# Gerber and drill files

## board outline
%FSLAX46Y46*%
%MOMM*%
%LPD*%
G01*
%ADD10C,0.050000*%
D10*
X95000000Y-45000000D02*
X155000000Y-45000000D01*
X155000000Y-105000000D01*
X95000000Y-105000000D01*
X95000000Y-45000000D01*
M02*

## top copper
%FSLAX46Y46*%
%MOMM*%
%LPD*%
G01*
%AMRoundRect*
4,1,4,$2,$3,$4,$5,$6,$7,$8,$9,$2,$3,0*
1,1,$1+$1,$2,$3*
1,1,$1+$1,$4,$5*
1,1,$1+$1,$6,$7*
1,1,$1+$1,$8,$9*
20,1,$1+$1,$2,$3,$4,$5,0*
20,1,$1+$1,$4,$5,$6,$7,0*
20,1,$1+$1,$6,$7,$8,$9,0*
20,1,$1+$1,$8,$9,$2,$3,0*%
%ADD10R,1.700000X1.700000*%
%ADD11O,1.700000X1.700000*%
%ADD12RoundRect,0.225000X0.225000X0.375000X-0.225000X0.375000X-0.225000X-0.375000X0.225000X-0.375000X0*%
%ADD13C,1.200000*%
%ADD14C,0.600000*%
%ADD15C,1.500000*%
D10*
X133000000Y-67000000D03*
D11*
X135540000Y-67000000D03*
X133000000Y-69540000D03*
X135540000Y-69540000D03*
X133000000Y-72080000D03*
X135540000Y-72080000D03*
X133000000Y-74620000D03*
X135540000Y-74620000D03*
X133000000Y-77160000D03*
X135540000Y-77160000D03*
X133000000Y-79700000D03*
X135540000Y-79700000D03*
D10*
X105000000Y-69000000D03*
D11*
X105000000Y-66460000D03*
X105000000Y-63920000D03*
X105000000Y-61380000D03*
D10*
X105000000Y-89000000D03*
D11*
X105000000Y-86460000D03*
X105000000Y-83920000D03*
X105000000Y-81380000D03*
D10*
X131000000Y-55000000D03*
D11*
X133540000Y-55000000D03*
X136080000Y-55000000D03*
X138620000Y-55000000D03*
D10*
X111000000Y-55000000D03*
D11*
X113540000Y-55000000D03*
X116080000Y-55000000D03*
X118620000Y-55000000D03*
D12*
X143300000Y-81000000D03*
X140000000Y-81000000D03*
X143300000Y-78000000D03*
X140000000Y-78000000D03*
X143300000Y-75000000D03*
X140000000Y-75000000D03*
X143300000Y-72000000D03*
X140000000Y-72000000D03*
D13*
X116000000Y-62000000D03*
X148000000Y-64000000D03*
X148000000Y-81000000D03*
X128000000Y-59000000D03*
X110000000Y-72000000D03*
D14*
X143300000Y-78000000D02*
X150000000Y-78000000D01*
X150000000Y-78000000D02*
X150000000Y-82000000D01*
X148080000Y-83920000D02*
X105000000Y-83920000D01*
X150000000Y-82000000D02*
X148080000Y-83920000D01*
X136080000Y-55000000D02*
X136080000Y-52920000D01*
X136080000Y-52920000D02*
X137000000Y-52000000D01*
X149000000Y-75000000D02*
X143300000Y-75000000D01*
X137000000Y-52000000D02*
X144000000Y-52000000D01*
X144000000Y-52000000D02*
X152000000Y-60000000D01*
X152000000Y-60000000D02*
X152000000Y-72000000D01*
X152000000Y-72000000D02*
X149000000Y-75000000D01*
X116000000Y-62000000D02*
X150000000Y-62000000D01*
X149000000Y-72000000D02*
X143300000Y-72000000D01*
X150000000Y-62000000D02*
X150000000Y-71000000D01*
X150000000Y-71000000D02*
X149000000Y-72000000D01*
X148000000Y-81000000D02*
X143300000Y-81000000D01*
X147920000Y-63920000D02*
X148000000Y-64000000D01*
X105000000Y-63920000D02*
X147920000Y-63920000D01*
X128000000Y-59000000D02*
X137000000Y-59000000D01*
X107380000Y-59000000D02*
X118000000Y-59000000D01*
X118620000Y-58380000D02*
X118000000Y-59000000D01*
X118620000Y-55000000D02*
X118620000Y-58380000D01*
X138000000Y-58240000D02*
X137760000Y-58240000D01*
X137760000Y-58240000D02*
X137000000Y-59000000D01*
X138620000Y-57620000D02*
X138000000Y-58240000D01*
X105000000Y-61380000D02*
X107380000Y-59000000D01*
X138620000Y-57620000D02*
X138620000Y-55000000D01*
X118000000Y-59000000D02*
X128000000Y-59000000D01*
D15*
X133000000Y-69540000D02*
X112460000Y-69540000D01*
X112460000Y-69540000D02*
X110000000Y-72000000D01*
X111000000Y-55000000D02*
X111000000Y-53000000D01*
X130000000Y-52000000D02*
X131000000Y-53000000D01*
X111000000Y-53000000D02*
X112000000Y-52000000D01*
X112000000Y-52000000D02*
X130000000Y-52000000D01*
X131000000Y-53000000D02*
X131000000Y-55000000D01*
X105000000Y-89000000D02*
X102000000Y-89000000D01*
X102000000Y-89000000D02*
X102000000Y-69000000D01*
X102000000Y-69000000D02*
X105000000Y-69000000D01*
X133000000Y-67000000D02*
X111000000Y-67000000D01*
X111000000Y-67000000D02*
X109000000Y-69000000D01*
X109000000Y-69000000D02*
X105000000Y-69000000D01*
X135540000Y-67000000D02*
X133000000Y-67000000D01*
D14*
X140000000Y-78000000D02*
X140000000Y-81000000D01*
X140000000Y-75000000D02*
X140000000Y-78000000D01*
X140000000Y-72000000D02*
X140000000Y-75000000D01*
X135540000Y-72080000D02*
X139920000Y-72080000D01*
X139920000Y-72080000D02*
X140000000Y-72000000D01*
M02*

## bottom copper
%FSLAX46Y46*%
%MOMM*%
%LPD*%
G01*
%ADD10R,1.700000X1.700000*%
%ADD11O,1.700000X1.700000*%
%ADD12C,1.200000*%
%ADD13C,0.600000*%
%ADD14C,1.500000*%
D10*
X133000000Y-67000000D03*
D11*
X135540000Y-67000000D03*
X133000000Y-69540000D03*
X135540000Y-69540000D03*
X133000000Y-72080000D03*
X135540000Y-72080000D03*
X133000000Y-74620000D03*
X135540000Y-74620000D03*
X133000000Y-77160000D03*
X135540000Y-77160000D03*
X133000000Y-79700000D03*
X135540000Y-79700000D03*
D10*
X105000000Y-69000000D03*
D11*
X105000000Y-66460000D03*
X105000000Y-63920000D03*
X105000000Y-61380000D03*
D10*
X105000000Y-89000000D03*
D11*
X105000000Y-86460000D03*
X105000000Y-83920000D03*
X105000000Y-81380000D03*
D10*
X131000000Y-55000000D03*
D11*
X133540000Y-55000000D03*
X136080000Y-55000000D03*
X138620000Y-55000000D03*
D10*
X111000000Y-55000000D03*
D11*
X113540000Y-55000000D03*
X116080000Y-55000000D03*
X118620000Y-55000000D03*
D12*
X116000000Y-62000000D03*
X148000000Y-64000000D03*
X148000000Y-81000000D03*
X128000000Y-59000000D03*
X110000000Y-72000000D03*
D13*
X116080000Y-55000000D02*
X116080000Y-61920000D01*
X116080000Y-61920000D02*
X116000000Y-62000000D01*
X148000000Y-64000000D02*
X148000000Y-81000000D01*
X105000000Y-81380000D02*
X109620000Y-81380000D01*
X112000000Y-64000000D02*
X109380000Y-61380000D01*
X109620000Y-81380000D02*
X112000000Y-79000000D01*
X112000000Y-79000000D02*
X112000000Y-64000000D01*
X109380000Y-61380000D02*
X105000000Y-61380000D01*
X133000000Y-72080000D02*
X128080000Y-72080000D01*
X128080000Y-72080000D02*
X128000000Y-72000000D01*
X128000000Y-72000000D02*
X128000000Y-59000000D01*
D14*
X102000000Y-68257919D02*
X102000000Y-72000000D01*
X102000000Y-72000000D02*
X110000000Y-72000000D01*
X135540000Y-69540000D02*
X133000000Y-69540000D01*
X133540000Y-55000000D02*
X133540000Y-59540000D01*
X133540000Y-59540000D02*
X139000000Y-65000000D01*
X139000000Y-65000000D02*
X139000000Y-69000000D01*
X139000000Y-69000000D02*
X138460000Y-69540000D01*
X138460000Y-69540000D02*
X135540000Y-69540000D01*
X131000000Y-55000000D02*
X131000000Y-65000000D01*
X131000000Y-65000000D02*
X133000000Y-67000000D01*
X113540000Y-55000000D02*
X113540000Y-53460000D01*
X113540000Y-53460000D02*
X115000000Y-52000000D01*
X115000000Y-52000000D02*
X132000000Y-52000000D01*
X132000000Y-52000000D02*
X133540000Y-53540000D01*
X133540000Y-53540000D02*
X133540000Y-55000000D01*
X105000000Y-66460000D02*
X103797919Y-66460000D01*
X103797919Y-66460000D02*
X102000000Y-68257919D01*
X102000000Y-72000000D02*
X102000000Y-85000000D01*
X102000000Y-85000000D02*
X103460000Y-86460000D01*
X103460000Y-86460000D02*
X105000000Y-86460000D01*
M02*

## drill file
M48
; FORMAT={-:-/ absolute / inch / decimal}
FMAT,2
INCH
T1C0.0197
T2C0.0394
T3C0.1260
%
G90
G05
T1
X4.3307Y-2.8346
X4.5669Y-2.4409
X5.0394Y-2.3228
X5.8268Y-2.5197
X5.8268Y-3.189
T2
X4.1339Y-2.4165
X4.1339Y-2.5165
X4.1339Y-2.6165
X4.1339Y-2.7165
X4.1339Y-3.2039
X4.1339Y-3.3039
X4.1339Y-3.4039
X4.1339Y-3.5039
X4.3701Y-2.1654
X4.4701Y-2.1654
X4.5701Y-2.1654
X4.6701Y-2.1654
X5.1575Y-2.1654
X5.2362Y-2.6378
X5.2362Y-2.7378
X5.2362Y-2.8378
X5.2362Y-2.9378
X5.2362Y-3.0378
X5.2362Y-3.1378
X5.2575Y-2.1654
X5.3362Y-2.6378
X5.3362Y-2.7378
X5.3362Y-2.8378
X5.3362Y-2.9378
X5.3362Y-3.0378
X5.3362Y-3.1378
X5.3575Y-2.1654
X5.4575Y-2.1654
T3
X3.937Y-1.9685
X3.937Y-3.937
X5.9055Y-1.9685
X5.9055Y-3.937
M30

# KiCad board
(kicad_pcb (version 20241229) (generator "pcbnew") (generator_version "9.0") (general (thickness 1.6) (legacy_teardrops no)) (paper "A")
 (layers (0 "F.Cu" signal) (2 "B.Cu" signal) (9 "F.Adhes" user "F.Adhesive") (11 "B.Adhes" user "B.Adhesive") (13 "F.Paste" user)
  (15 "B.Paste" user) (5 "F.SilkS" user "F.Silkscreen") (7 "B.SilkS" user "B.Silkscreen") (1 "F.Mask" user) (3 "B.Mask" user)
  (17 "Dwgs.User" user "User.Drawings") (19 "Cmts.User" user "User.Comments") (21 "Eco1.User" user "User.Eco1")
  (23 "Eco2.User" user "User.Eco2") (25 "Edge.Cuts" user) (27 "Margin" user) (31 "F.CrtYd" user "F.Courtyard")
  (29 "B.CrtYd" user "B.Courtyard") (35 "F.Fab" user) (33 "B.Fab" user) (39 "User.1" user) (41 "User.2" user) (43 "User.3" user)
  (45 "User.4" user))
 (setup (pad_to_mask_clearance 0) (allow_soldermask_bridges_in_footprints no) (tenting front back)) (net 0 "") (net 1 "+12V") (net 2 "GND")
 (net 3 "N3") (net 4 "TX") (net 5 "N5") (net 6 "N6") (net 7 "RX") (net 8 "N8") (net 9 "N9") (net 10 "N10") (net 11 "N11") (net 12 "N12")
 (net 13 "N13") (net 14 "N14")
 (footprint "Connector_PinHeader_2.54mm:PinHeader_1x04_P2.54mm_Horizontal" (layer "F.Cu") (at 131 55 90)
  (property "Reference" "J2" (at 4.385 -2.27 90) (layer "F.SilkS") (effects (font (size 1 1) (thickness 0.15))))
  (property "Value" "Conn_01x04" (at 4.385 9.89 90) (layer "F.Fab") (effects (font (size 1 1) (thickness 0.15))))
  (pad "1" thru_hole rect (at 0 0 90) (size 1.7 1.7) (drill 1) (layers "*.Cu" "*.Mask") (remove_unused_layers no) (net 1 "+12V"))
  (pad "2" thru_hole oval (at 0 2.54 90) (size 1.7 1.7) (drill 1) (layers "*.Cu" "*.Mask") (remove_unused_layers no) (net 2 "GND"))
  (pad "3" thru_hole oval (at 0 5.08 90) (size 1.7 1.7) (drill 1) (layers "*.Cu" "*.Mask") (remove_unused_layers no) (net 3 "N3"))
  (pad "4" thru_hole oval (at 0 7.62 90) (size 1.7 1.7) (drill 1) (layers "*.Cu" "*.Mask") (remove_unused_layers no) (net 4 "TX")))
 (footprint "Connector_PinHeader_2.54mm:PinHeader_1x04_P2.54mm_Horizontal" (layer "F.Cu") (at 105 89 180)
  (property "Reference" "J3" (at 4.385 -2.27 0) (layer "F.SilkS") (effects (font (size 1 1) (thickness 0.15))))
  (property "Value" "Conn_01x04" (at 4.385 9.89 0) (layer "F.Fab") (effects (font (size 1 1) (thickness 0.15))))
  (pad "1" thru_hole rect (at 0 0 180) (size 1.7 1.7) (drill 1) (layers "*.Cu" "*.Mask") (remove_unused_layers no) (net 1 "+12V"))
  (pad "2" thru_hole oval (at 0 2.54 180) (size 1.7 1.7) (drill 1) (layers "*.Cu" "*.Mask") (remove_unused_layers no) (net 2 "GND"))
  (pad "3" thru_hole oval (at 0 5.08 180) (size 1.7 1.7) (drill 1) (layers "*.Cu" "*.Mask") (remove_unused_layers no) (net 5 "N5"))
  (pad "4" thru_hole oval (at 0 7.62 180) (size 1.7 1.7) (drill 1) (layers "*.Cu" "*.Mask") (remove_unused_layers no) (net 4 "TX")))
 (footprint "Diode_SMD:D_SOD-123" (layer "F.Cu") (at 141.65 81 180)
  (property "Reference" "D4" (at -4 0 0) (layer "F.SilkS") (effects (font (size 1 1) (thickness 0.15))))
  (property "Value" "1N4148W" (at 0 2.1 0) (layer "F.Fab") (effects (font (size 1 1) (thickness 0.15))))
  (pad "1" smd roundrect (at -1.65 0 180) (size 0.9 1.2) (layers "F.Cu" "F.Mask" "F.Paste") (roundrect_rratio 0.25) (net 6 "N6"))
  (pad "2" smd roundrect (at 1.65 0 180) (size 0.9 1.2) (layers "F.Cu" "F.Mask" "F.Paste") (roundrect_rratio 0.25) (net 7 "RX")))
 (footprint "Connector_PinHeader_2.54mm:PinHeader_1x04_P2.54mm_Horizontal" (layer "F.Cu") (at 105 69 180)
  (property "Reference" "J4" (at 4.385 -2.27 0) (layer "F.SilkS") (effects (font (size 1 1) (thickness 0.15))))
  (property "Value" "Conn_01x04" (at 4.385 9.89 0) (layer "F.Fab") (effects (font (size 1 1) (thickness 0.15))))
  (pad "1" thru_hole rect (at 0 0 180) (size 1.7 1.7) (drill 1) (layers "*.Cu" "*.Mask") (remove_unused_layers no) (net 1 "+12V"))
  (pad "2" thru_hole oval (at 0 2.54 180) (size 1.7 1.7) (drill 1) (layers "*.Cu" "*.Mask") (remove_unused_layers no) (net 2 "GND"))
  (pad "3" thru_hole oval (at 0 5.08 180) (size 1.7 1.7) (drill 1) (layers "*.Cu" "*.Mask") (remove_unused_layers no) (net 6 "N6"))
  (pad "4" thru_hole oval (at 0 7.62 180) (size 1.7 1.7) (drill 1) (layers "*.Cu" "*.Mask") (remove_unused_layers no) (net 4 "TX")))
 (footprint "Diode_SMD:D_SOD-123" (layer "F.Cu") (at 141.65 75 180)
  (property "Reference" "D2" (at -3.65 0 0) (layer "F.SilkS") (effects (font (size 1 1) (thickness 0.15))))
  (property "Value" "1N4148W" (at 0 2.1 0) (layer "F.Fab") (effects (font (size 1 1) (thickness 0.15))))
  (pad "1" smd roundrect (at -1.65 0 180) (size 0.9 1.2) (layers "F.Cu" "F.Mask" "F.Paste") (roundrect_rratio 0.25) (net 3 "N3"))
  (pad "2" smd roundrect (at 1.65 0 180) (size 0.9 1.2) (layers "F.Cu" "F.Mask" "F.Paste") (roundrect_rratio 0.25) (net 7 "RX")))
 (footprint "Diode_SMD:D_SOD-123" (layer "F.Cu") (at 141.65 72 180)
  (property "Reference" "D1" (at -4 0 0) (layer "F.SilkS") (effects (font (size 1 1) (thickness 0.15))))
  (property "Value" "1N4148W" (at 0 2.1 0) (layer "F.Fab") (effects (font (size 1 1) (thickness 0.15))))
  (pad "1" smd roundrect (at -1.65 0 180) (size 0.9 1.2) (layers "F.Cu" "F.Mask" "F.Paste") (roundrect_rratio 0.25) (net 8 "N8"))
  (pad "2" smd roundrect (at 1.65 0 180) (size 0.9 1.2) (layers "F.Cu" "F.Mask" "F.Paste") (roundrect_rratio 0.25) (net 7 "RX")))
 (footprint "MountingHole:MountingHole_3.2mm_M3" (layer "F.Cu") (at 150 100)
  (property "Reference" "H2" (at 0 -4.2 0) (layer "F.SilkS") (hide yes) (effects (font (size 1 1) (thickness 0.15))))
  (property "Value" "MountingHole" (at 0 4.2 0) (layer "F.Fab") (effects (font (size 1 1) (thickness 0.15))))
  (pad "" np_thru_hole circle (at 0 0) (size 3.2 3.2) (drill 3.2) (layers "*.Cu" "*.Mask")))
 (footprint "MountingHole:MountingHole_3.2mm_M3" (layer "F.Cu") (at 100 50)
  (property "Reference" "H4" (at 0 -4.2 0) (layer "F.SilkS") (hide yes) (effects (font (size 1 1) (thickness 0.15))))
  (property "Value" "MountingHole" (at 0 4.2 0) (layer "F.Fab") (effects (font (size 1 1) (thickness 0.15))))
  (pad "" np_thru_hole circle (at 0 0) (size 3.2 3.2) (drill 3.2) (layers "*.Cu" "*.Mask")))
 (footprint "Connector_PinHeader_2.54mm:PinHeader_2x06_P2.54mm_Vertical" (layer "F.Cu") (at 133 67)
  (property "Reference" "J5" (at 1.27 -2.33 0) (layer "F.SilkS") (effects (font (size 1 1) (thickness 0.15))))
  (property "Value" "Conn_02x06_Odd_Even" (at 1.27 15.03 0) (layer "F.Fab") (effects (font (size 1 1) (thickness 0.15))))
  (pad "1" thru_hole rect (at 0 0) (size 1.7 1.7) (drill 1) (layers "*.Cu" "*.Mask") (remove_unused_layers no) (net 1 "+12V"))
  (pad "2" thru_hole oval (at 2.54 0) (size 1.7 1.7) (drill 1) (layers "*.Cu" "*.Mask") (remove_unused_layers no) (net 1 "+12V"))
  (pad "3" thru_hole oval (at 0 2.54) (size 1.7 1.7) (drill 1) (layers "*.Cu" "*.Mask") (remove_unused_layers no) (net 2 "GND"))
  (pad "4" thru_hole oval (at 2.54 2.54) (size 1.7 1.7) (drill 1) (layers "*.Cu" "*.Mask") (remove_unused_layers no) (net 2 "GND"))
  (pad "5" thru_hole oval (at 0 5.08) (size 1.7 1.7) (drill 1) (layers "*.Cu" "*.Mask") (remove_unused_layers no) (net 4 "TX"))
  (pad "6" thru_hole oval (at 2.54 5.08) (size 1.7 1.7) (drill 1) (layers "*.Cu" "*.Mask") (remove_unused_layers no) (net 7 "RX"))
  (pad "7" thru_hole oval (at 0 7.62) (size 1.7 1.7) (drill 1) (layers "*.Cu" "*.Mask") (remove_unused_layers no) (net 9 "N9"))
  (pad "8" thru_hole oval (at 2.54 7.62) (size 1.7 1.7) (drill 1) (layers "*.Cu" "*.Mask") (remove_unused_layers no) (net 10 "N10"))
  (pad "9" thru_hole oval (at 0 10.16) (size 1.7 1.7) (drill 1) (layers "*.Cu" "*.Mask") (remove_unused_layers no) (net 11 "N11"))
  (pad "10" thru_hole oval (at 2.54 10.16) (size 1.7 1.7) (drill 1) (layers "*.Cu" "*.Mask") (remove_unused_layers no) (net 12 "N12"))
  (pad "11" thru_hole oval (at 0 12.7) (size 1.7 1.7) (drill 1) (layers "*.Cu" "*.Mask") (remove_unused_layers no) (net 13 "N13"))
  (pad "12" thru_hole oval (at 2.54 12.7) (size 1.7 1.7) (drill 1) (layers "*.Cu" "*.Mask") (remove_unused_layers no) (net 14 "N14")))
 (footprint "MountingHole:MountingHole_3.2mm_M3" (layer "F.Cu") (at 100 100)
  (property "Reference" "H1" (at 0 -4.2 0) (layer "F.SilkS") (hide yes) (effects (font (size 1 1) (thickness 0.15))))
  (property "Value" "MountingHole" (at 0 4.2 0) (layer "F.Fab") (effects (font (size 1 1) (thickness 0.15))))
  (pad "" np_thru_hole circle (at 0 0) (size 3.2 3.2) (drill 3.2) (layers "*.Cu" "*.Mask")))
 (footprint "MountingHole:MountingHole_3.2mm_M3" (layer "F.Cu") (at 150 50)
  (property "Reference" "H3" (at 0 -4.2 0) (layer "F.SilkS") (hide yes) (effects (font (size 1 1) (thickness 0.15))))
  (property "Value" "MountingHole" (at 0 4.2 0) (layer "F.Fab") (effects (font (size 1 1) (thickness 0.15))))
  (pad "" np_thru_hole circle (at 0 0) (size 3.2 3.2) (drill 3.2) (layers "*.Cu" "*.Mask")))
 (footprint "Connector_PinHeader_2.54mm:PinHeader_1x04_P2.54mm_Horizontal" (layer "F.Cu") (at 111 55 90)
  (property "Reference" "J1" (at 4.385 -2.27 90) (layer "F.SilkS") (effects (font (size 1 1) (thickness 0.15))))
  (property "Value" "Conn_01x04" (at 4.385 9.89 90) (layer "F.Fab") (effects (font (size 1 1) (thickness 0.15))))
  (pad "1" thru_hole rect (at 0 0 90) (size 1.7 1.7) (drill 1) (layers "*.Cu" "*.Mask") (remove_unused_layers no) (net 1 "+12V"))
  (pad "2" thru_hole oval (at 0 2.54 90) (size 1.7 1.7) (drill 1) (layers "*.Cu" "*.Mask") (remove_unused_layers no) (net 2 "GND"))
  (pad "3" thru_hole oval (at 0 5.08 90) (size 1.7 1.7) (drill 1) (layers "*.Cu" "*.Mask") (remove_unused_layers no) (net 8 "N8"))
  (pad "4" thru_hole oval (at 0 7.62 90) (size 1.7 1.7) (drill 1) (layers "*.Cu" "*.Mask") (remove_unused_layers no) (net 4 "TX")))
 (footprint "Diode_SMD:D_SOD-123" (layer "F.Cu") (at 141.65 78 180)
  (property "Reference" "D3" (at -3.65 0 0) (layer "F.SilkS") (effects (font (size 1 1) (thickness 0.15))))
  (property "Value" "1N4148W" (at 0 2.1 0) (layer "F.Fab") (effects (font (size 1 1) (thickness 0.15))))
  (pad "1" smd roundrect (at -1.65 0 180) (size 0.9 1.2) (layers "F.Cu" "F.Mask" "F.Paste") (roundrect_rratio 0.25) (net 5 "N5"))
  (pad "2" smd roundrect (at 1.65 0 180) (size 0.9 1.2) (layers "F.Cu" "F.Mask" "F.Paste") (roundrect_rratio 0.25) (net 7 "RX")))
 (gr_rect (start 95 45) (end 155 105) (stroke (width 0.05) (type default)) (fill no) (layer "Edge.Cuts"))
 (segment (start 116 62) (end 150 62) (width 0.6) (layer "F.Cu") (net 8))
 (segment (start 150 62) (end 150 71) (width 0.6) (layer "F.Cu") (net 8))
 (segment (start 149 72) (end 143.3 72) (width 0.6) (layer "F.Cu") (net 8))
 (segment (start 150 71) (end 149 72) (width 0.6) (layer "F.Cu") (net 8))
 (via (at 116 62) (size 1.2) (drill 0.5) (layers "F.Cu" "B.Cu") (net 8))
 (segment (start 116.08 55) (end 116.08 61.92) (width 0.6) (layer "B.Cu") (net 8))
 (segment (start 116.08 61.92) (end 116 62) (width 0.6) (layer "B.Cu") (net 8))
 (segment (start 140 75) (end 140 78) (width 0.6) (layer "F.Cu") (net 7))
 (segment (start 140 78) (end 140 81) (width 0.6) (layer "F.Cu") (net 7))
 (segment (start 135.54 72.08) (end 139.92 72.08) (width 0.6) (layer "F.Cu") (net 7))
 (segment (start 139.92 72.08) (end 140 72) (width 0.6) (layer "F.Cu") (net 7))
 (segment (start 140 72) (end 140 75) (width 0.6) (layer "F.Cu") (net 7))
 (segment (start 136.08 55) (end 136.08 52.92) (width 0.6) (layer "F.Cu") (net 3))
 (segment (start 152 72) (end 149 75) (width 0.6) (layer "F.Cu") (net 3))
 (segment (start 136.08 52.92) (end 137 52) (width 0.6) (layer "F.Cu") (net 3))
 (segment (start 144 52) (end 152 60) (width 0.6) (layer "F.Cu") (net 3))
 (segment (start 152 60) (end 152 72) (width 0.6) (layer "F.Cu") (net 3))
 (segment (start 137 52) (end 144 52) (width 0.6) (layer "F.Cu") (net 3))
 (segment (start 149 75) (end 143.3 75) (width 0.6) (layer "F.Cu") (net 3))
 (segment (start 150 82) (end 148.08 83.92) (width 0.6) (layer "F.Cu") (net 5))
 (segment (start 150 78) (end 150 82) (width 0.6) (layer "F.Cu") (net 5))
 (segment (start 148.08 83.92) (end 105 83.92) (width 0.6) (layer "F.Cu") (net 5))
 (segment (start 143.3 78) (end 150 78) (width 0.6) (layer "F.Cu") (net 5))
 (segment (start 147.92 63.92) (end 148 64) (width 0.6) (layer "F.Cu") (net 6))
 (segment (start 105 63.92) (end 147.92 63.92) (width 0.6) (layer "F.Cu") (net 6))
 (segment (start 148 81) (end 143.3 81) (width 0.6) (layer "F.Cu") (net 6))
 (via (at 148 64) (size 1.2) (drill 0.5) (layers "F.Cu" "B.Cu") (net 6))
 (via (at 148 81) (size 1.2) (drill 0.5) (layers "F.Cu" "B.Cu") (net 6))
 (segment (start 148 64) (end 148 81) (width 0.6) (layer "B.Cu") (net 6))
 (segment (start 105 89) (end 102 89) (width 1.5) (layer "F.Cu") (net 1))
 (segment (start 135.54 67) (end 133 67) (width 1.5) (layer "F.Cu") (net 1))
 (segment (start 102 69) (end 105 69) (width 1.5) (layer "F.Cu") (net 1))
 (segment (start 102 89) (end 102 69) (width 1.5) (layer "F.Cu") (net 1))
 (segment (start 131 53) (end 131 55) (width 1.5) (layer "F.Cu") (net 1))
 (segment (start 112 52) (end 130 52) (width 1.5) (layer "F.Cu") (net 1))
 (segment (start 133 67) (end 111 67) (width 1.5) (layer "F.Cu") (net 1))
 (segment (start 111 67) (end 109 69) (width 1.5) (layer "F.Cu") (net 1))
 (segment (start 111 55) (end 111 53) (width 1.5) (layer "F.Cu") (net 1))
 (segment (start 109 69) (end 105 69) (width 1.5) (layer "F.Cu") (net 1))
 (segment (start 130 52) (end 131 53) (width 1.5) (layer "F.Cu") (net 1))
 (segment (start 111 53) (end 112 52) (width 1.5) (layer "F.Cu") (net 1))
 (segment (start 131 55) (end 131 65) (width 1.5) (layer "B.Cu") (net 1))
 (segment (start 131 65) (end 133 67) (width 1.5) (layer "B.Cu") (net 1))
 (segment (start 138.62 57.62) (end 138.62 55) (width 0.6) (layer "F.Cu") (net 4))
 (segment (start 105 61.38) (end 107.38 59) (width 0.6) (layer "F.Cu") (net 4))
 (segment (start 138.62 57.62) (end 138 58.24) (width 0.6) (layer "F.Cu") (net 4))
 (segment (start 137.76 58.24) (end 137 59) (width 0.6) (layer "F.Cu") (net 4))
 (segment (start 138 58.24) (end 137.76 58.24) (width 0.6) (layer "F.Cu") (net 4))
 (segment (start 118.62 55) (end 118.62 58.38) (width 0.6) (layer "F.Cu") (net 4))
 (segment (start 118 59) (end 128 59) (width 0.6) (layer "F.Cu") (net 4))
 (segment (start 128 59) (end 137 59) (width 0.6) (layer "F.Cu") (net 4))
 (segment (start 107.38 59) (end 118 59) (width 0.6) (layer "F.Cu") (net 4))
 (segment (start 118.62 58.38) (end 118 59) (width 0.6) (layer "F.Cu") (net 4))
 (via (at 128 59) (size 1.2) (drill 0.5) (layers "F.Cu" "B.Cu") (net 4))
 (segment (start 112 79) (end 112 64) (width 0.6) (layer "B.Cu") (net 4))
 (segment (start 105 81.38) (end 109.62 81.38) (width 0.6) (layer "B.Cu") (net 4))
 (segment (start 128 72) (end 128 59) (width 0.6) (layer "B.Cu") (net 4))
 (segment (start 109.62 81.38) (end 112 79) (width 0.6) (layer "B.Cu") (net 4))
 (segment (start 112 64) (end 109.38 61.38) (width 0.6) (layer "B.Cu") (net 4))
 (segment (start 133 72.08) (end 128.08 72.08) (width 0.6) (layer "B.Cu") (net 4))
 (segment (start 109.38 61.38) (end 105 61.38) (width 0.6) (layer "B.Cu") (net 4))
 (segment (start 128.08 72.08) (end 128 72) (width 0.6) (layer "B.Cu") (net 4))
 (segment (start 133 69.54) (end 112.46 69.54) (width 1.5) (layer "F.Cu") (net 2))
 (segment (start 112.46 69.54) (end 110 72) (width 1.5) (layer "F.Cu") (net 2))
 (via (at 110 72) (size 1.2) (drill 0.5) (layers "F.Cu" "B.Cu") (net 2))
 (segment (start 133.54 53.54) (end 133.54 55) (width 1.5) (layer "B.Cu") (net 2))
 (segment (start 102 72) (end 102 85) (width 1.5) (layer "B.Cu") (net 2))
 (segment (start 103.797919 66.46) (end 102 68.257919) (width 1.5) (layer "B.Cu") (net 2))
 (segment (start 103.46 86.46) (end 105 86.46) (width 1.5) (layer "B.Cu") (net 2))
 (segment (start 102 72) (end 110 72) (width 1.5) (layer "B.Cu") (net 2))
 (segment (start 132 52) (end 133.54 53.54) (width 1.5) (layer "B.Cu") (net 2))
 (segment (start 113.54 53.46) (end 115 52) (width 1.5) (layer "B.Cu") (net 2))
 (segment (start 102 85) (end 103.46 86.46) (width 1.5) (layer "B.Cu") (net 2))
 (segment (start 135.54 69.54) (end 133 69.54) (width 1.5) (layer "B.Cu") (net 2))
 (segment (start 102 68.257919) (end 102 72) (width 1.5) (layer "B.Cu") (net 2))
 (segment (start 133.54 59.54) (end 139 65) (width 1.5) (layer "B.Cu") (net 2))
 (segment (start 139 65) (end 139 69) (width 1.5) (layer "B.Cu") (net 2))
 (segment (start 105 66.46) (end 103.797919 66.46) (width 1.5) (layer "B.Cu") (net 2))
 (segment (start 138.46 69.54) (end 135.54 69.54) (width 1.5) (layer "B.Cu") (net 2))
 (segment (start 139 69) (end 138.46 69.54) (width 1.5) (layer "B.Cu") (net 2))
 (segment (start 133.54 55) (end 133.54 59.54) (width 1.5) (layer "B.Cu") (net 2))
 (segment (start 113.54 55) (end 113.54 53.46) (width 1.5) (layer "B.Cu") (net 2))
 (segment (start 115 52) (end 132 52) (width 1.5) (layer "B.Cu") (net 2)))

